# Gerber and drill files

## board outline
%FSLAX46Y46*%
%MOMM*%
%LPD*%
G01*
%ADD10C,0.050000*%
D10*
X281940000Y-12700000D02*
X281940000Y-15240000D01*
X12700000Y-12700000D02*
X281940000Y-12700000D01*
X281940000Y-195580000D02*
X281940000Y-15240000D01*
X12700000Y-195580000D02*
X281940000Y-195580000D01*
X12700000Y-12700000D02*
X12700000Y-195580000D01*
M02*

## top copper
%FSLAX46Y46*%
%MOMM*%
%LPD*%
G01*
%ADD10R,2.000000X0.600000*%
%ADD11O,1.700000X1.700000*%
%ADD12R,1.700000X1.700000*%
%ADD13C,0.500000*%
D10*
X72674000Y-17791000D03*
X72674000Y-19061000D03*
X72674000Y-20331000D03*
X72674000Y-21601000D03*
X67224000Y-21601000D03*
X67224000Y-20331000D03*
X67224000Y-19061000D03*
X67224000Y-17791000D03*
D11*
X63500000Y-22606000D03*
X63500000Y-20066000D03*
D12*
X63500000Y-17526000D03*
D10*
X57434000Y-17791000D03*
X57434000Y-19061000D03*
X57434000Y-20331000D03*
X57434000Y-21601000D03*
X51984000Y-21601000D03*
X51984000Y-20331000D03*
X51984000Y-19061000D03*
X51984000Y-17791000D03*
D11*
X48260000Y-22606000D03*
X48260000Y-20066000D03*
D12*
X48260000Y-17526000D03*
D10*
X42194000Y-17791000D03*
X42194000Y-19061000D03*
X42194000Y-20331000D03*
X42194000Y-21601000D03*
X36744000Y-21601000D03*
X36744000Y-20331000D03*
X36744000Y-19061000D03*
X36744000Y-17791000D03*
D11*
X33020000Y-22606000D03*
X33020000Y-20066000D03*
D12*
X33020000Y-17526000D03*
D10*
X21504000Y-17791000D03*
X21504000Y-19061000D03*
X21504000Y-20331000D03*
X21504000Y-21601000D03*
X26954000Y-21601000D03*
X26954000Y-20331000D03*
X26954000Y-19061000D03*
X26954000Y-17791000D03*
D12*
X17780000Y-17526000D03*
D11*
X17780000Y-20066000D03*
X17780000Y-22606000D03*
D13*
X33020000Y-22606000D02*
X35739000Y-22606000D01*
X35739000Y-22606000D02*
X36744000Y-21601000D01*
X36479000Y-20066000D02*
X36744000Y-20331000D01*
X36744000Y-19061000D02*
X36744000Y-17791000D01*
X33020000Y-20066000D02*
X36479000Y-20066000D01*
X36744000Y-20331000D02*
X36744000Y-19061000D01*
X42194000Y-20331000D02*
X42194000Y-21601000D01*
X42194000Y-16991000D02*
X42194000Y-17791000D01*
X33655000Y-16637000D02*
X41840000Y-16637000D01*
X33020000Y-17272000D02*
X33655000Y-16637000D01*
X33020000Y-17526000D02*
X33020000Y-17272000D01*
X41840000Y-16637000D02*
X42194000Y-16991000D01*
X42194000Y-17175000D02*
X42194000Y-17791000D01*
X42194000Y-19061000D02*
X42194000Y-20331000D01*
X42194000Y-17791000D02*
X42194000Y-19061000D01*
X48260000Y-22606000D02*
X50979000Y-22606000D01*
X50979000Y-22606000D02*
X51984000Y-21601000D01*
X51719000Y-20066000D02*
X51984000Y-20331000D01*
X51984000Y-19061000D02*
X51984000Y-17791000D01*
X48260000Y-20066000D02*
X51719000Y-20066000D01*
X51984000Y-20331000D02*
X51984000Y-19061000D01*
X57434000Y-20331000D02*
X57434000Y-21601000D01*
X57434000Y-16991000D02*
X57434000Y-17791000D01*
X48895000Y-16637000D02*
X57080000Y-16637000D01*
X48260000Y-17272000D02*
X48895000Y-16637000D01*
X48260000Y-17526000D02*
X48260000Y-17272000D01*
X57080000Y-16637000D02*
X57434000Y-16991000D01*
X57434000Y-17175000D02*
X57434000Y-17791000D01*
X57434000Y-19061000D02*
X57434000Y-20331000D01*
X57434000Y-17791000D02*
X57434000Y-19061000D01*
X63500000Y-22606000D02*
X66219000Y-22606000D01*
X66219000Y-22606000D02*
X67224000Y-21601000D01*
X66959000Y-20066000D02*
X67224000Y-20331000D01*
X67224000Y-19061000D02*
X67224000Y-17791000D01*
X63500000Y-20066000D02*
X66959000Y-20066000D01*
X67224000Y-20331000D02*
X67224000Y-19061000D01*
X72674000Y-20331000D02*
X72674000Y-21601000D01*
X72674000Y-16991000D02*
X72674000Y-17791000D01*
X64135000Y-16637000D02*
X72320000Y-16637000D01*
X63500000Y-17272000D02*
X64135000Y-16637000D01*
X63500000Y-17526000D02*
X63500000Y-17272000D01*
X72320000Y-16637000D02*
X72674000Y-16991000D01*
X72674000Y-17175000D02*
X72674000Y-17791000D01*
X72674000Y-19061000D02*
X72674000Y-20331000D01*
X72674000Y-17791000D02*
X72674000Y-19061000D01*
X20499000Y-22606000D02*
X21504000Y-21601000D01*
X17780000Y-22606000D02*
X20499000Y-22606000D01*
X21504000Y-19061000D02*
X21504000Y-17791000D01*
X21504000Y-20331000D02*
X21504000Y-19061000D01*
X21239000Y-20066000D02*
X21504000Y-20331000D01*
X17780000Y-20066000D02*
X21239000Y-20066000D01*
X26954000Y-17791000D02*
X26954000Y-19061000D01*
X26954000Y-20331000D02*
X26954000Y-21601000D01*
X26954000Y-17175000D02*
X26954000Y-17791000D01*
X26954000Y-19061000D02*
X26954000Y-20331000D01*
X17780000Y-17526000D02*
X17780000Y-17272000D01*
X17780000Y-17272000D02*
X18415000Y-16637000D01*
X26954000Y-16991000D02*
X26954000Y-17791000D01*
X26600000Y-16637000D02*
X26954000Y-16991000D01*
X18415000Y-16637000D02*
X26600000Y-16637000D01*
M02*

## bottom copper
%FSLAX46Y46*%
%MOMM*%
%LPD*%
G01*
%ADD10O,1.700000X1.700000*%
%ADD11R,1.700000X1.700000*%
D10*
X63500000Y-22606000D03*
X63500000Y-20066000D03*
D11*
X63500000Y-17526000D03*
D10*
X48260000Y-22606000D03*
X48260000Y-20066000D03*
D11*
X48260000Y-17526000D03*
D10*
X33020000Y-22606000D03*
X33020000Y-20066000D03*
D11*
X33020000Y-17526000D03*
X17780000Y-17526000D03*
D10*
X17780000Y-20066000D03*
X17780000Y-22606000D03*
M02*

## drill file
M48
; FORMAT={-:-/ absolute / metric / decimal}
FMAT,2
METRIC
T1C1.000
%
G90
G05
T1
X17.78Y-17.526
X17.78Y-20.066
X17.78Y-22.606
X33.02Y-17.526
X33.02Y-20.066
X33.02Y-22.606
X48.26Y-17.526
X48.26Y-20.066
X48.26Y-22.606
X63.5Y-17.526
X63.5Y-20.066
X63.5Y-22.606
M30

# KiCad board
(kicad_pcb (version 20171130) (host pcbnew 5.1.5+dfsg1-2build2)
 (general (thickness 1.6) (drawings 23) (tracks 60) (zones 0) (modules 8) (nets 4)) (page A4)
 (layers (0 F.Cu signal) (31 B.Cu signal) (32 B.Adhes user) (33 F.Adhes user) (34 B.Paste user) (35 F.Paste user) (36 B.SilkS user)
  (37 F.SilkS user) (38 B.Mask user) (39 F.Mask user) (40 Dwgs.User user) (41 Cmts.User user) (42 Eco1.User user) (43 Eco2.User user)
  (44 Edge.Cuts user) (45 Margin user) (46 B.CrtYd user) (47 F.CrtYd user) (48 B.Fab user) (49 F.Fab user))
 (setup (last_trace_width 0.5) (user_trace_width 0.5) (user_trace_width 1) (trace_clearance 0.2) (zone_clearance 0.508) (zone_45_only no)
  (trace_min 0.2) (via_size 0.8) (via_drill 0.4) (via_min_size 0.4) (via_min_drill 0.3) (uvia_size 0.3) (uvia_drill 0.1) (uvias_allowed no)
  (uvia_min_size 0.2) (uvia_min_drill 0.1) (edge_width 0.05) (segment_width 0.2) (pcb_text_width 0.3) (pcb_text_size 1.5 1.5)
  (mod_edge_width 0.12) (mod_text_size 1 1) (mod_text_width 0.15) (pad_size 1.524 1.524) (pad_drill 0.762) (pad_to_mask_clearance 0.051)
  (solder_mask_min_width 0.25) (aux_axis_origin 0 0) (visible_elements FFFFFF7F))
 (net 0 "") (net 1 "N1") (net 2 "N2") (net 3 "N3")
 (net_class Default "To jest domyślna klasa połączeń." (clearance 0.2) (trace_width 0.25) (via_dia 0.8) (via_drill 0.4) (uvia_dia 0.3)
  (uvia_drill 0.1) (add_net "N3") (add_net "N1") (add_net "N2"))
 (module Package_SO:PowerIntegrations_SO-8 (layer F.Cu) (at 69.949 19.696)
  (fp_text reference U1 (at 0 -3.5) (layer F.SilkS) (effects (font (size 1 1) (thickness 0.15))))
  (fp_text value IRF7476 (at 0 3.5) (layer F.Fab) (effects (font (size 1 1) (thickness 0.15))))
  (pad 8 smd rect (at 2.725 -1.905) (size 2 0.6) (layers F.Cu F.Paste F.Mask))
  (pad 7 smd rect (at 2.725 -0.635) (size 2 0.6) (layers F.Cu F.Paste F.Mask))
  (pad 6 smd rect (at 2.725 0.635) (size 2 0.6) (layers F.Cu F.Paste F.Mask))
  (pad 5 smd rect (at 2.725 1.905) (size 2 0.6) (layers F.Cu F.Paste F.Mask))
  (pad 4 smd rect (at -2.725 1.905) (size 2 0.6) (layers F.Cu F.Paste F.Mask))
  (pad 3 smd rect (at -2.725 0.635) (size 2 0.6) (layers F.Cu F.Paste F.Mask))
  (pad 2 smd rect (at -2.725 -0.635) (size 2 0.6) (layers F.Cu F.Paste F.Mask))
  (pad 1 smd rect (at -2.725 -1.905) (size 2 0.6) (layers F.Cu F.Paste F.Mask)))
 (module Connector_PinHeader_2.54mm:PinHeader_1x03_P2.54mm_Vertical (layer B.Cu) (at 63.5 17.526 180)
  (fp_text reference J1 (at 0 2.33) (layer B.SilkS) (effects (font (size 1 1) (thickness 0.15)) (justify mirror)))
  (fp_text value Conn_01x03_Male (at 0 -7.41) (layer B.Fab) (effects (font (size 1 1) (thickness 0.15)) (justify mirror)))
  (pad 3 thru_hole oval (at 0 -5.08 180) (size 1.7 1.7) (drill 1) (layers *.Cu *.Mask))
  (pad 2 thru_hole oval (at 0 -2.54 180) (size 1.7 1.7) (drill 1) (layers *.Cu *.Mask))
  (pad 1 thru_hole rect (at 0 0 180) (size 1.7 1.7) (drill 1) (layers *.Cu *.Mask)))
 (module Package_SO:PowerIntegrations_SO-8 (layer F.Cu) (at 54.709 19.696)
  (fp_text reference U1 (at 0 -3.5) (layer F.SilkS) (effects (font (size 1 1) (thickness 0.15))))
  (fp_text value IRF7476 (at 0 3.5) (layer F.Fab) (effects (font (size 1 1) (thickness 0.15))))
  (pad 8 smd rect (at 2.725 -1.905) (size 2 0.6) (layers F.Cu F.Paste F.Mask))
  (pad 7 smd rect (at 2.725 -0.635) (size 2 0.6) (layers F.Cu F.Paste F.Mask))
  (pad 6 smd rect (at 2.725 0.635) (size 2 0.6) (layers F.Cu F.Paste F.Mask))
  (pad 5 smd rect (at 2.725 1.905) (size 2 0.6) (layers F.Cu F.Paste F.Mask))
  (pad 4 smd rect (at -2.725 1.905) (size 2 0.6) (layers F.Cu F.Paste F.Mask))
  (pad 3 smd rect (at -2.725 0.635) (size 2 0.6) (layers F.Cu F.Paste F.Mask))
  (pad 2 smd rect (at -2.725 -0.635) (size 2 0.6) (layers F.Cu F.Paste F.Mask))
  (pad 1 smd rect (at -2.725 -1.905) (size 2 0.6) (layers F.Cu F.Paste F.Mask)))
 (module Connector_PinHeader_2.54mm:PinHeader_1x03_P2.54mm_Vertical (layer B.Cu) (at 48.26 17.526 180)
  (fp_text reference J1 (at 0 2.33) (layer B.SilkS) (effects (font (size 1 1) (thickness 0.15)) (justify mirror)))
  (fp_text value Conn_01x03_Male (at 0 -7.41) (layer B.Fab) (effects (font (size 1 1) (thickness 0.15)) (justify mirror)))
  (pad 3 thru_hole oval (at 0 -5.08 180) (size 1.7 1.7) (drill 1) (layers *.Cu *.Mask))
  (pad 2 thru_hole oval (at 0 -2.54 180) (size 1.7 1.7) (drill 1) (layers *.Cu *.Mask))
  (pad 1 thru_hole rect (at 0 0 180) (size 1.7 1.7) (drill 1) (layers *.Cu *.Mask)))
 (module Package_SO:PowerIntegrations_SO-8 (layer F.Cu) (at 39.469 19.696)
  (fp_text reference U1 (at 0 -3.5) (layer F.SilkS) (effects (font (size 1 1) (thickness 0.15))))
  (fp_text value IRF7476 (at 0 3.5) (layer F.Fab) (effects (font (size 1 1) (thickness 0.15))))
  (pad 8 smd rect (at 2.725 -1.905) (size 2 0.6) (layers F.Cu F.Paste F.Mask))
  (pad 7 smd rect (at 2.725 -0.635) (size 2 0.6) (layers F.Cu F.Paste F.Mask))
  (pad 6 smd rect (at 2.725 0.635) (size 2 0.6) (layers F.Cu F.Paste F.Mask))
  (pad 5 smd rect (at 2.725 1.905) (size 2 0.6) (layers F.Cu F.Paste F.Mask))
  (pad 4 smd rect (at -2.725 1.905) (size 2 0.6) (layers F.Cu F.Paste F.Mask))
  (pad 3 smd rect (at -2.725 0.635) (size 2 0.6) (layers F.Cu F.Paste F.Mask))
  (pad 2 smd rect (at -2.725 -0.635) (size 2 0.6) (layers F.Cu F.Paste F.Mask))
  (pad 1 smd rect (at -2.725 -1.905) (size 2 0.6) (layers F.Cu F.Paste F.Mask)))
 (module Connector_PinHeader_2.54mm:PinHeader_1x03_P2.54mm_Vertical (layer B.Cu) (at 33.02 17.526 180)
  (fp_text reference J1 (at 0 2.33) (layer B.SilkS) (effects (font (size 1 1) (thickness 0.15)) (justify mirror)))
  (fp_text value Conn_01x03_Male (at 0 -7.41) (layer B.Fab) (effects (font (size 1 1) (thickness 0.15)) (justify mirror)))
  (pad 3 thru_hole oval (at 0 -5.08 180) (size 1.7 1.7) (drill 1) (layers *.Cu *.Mask))
  (pad 2 thru_hole oval (at 0 -2.54 180) (size 1.7 1.7) (drill 1) (layers *.Cu *.Mask))
  (pad 1 thru_hole rect (at 0 0 180) (size 1.7 1.7) (drill 1) (layers *.Cu *.Mask)))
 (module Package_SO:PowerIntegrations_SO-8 (layer F.Cu) (at 24.229 19.696)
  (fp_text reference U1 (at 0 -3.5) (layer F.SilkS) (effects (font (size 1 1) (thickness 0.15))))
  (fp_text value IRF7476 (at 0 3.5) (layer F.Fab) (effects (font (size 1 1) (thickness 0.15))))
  (pad 1 smd rect (at -2.725 -1.905) (size 2 0.6) (layers F.Cu F.Paste F.Mask) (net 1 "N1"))
  (pad 2 smd rect (at -2.725 -0.635) (size 2 0.6) (layers F.Cu F.Paste F.Mask) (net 1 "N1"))
  (pad 3 smd rect (at -2.725 0.635) (size 2 0.6) (layers F.Cu F.Paste F.Mask) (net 1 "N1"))
  (pad 4 smd rect (at -2.725 1.905) (size 2 0.6) (layers F.Cu F.Paste F.Mask) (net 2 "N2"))
  (pad 5 smd rect (at 2.725 1.905) (size 2 0.6) (layers F.Cu F.Paste F.Mask) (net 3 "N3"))
  (pad 6 smd rect (at 2.725 0.635) (size 2 0.6) (layers F.Cu F.Paste F.Mask) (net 3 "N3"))
  (pad 7 smd rect (at 2.725 -0.635) (size 2 0.6) (layers F.Cu F.Paste F.Mask) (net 3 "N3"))
  (pad 8 smd rect (at 2.725 -1.905) (size 2 0.6) (layers F.Cu F.Paste F.Mask) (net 3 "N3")))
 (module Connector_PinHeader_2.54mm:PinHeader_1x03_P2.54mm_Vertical (layer B.Cu) (at 17.78 17.526 180)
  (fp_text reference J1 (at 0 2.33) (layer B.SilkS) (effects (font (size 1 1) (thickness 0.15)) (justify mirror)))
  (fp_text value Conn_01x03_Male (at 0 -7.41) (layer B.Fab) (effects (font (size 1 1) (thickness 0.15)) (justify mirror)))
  (pad 1 thru_hole rect (at 0 0 180) (size 1.7 1.7) (drill 1) (layers *.Cu *.Mask) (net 3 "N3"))
  (pad 2 thru_hole oval (at 0 -2.54 180) (size 1.7 1.7) (drill 1) (layers *.Cu *.Mask) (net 1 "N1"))
  (pad 3 thru_hole oval (at 0 -5.08 180) (size 1.7 1.7) (drill 1) (layers *.Cu *.Mask) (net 2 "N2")))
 (gr_line (start 281.94 12.7) (end 281.94 15.24) (layer Edge.Cuts) (width 0.05))
 (gr_line (start 12.7 12.7) (end 281.94 12.7) (layer Edge.Cuts) (width 0.05))
 (gr_line (start 281.94 195.58) (end 281.94 15.24) (layer Edge.Cuts) (width 0.05))
 (gr_line (start 12.7 195.58) (end 281.94 195.58) (layer Edge.Cuts) (width 0.05))
 (gr_line (start 12.7 12.7) (end 12.7 195.58) (layer Edge.Cuts) (width 0.05))
 (segment (start 33.02 22.606) (end 35.739 22.606) (width 0.5) (layer F.Cu) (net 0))
 (segment (start 35.739 22.606) (end 36.744 21.601) (width 0.5) (layer F.Cu) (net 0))
 (segment (start 36.479 20.066) (end 36.744 20.331) (width 0.5) (layer F.Cu) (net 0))
 (segment (start 36.744 19.061) (end 36.744 17.791) (width 0.5) (layer F.Cu) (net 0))
 (segment (start 33.02 20.066) (end 36.479 20.066) (width 0.5) (layer F.Cu) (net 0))
 (segment (start 36.744 20.331) (end 36.744 19.061) (width 0.5) (layer F.Cu) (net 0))
 (segment (start 42.194 20.331) (end 42.194 21.601) (width 0.5) (layer F.Cu) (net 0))
 (segment (start 42.194 16.991) (end 42.194 17.791) (width 0.5) (layer F.Cu) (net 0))
 (segment (start 33.655 16.637) (end 41.84 16.637) (width 0.5) (layer F.Cu) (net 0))
 (segment (start 33.02 17.272) (end 33.655 16.637) (width 0.5) (layer F.Cu) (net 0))
 (segment (start 33.02 17.526) (end 33.02 17.272) (width 0.5) (layer F.Cu) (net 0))
 (segment (start 41.84 16.637) (end 42.194 16.991) (width 0.5) (layer F.Cu) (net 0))
 (segment (start 42.194 17.175) (end 42.194 17.791) (width 0.5) (layer F.Cu) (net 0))
 (segment (start 42.194 19.061) (end 42.194 20.331) (width 0.5) (layer F.Cu) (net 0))
 (segment (start 42.194 17.791) (end 42.194 19.061) (width 0.5) (layer F.Cu) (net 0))
 (segment (start 48.26 22.606) (end 50.979 22.606) (width 0.5) (layer F.Cu) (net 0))
 (segment (start 50.979 22.606) (end 51.984 21.601) (width 0.5) (layer F.Cu) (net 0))
 (segment (start 51.719 20.066) (end 51.984 20.331) (width 0.5) (layer F.Cu) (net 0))
 (segment (start 51.984 19.061) (end 51.984 17.791) (width 0.5) (layer F.Cu) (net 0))
 (segment (start 48.26 20.066) (end 51.719 20.066) (width 0.5) (layer F.Cu) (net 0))
 (segment (start 51.984 20.331) (end 51.984 19.061) (width 0.5) (layer F.Cu) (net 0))
 (segment (start 57.434 20.331) (end 57.434 21.601) (width 0.5) (layer F.Cu) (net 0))
 (segment (start 57.434 16.991) (end 57.434 17.791) (width 0.5) (layer F.Cu) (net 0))
 (segment (start 48.895 16.637) (end 57.08 16.637) (width 0.5) (layer F.Cu) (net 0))
 (segment (start 48.26 17.272) (end 48.895 16.637) (width 0.5) (layer F.Cu) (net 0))
 (segment (start 48.26 17.526) (end 48.26 17.272) (width 0.5) (layer F.Cu) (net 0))
 (segment (start 57.08 16.637) (end 57.434 16.991) (width 0.5) (layer F.Cu) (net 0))
 (segment (start 57.434 17.175) (end 57.434 17.791) (width 0.5) (layer F.Cu) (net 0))
 (segment (start 57.434 19.061) (end 57.434 20.331) (width 0.5) (layer F.Cu) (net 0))
 (segment (start 57.434 17.791) (end 57.434 19.061) (width 0.5) (layer F.Cu) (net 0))
 (segment (start 63.5 22.606) (end 66.219 22.606) (width 0.5) (layer F.Cu) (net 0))
 (segment (start 66.219 22.606) (end 67.224 21.601) (width 0.5) (layer F.Cu) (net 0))
 (segment (start 66.959 20.066) (end 67.224 20.331) (width 0.5) (layer F.Cu) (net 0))
 (segment (start 67.224 19.061) (end 67.224 17.791) (width 0.5) (layer F.Cu) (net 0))
 (segment (start 63.5 20.066) (end 66.959 20.066) (width 0.5) (layer F.Cu) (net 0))
 (segment (start 67.224 20.331) (end 67.224 19.061) (width 0.5) (layer F.Cu) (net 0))
 (segment (start 72.674 20.331) (end 72.674 21.601) (width 0.5) (layer F.Cu) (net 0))
 (segment (start 72.674 16.991) (end 72.674 17.791) (width 0.5) (layer F.Cu) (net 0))
 (segment (start 64.135 16.637) (end 72.32 16.637) (width 0.5) (layer F.Cu) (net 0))
 (segment (start 63.5 17.272) (end 64.135 16.637) (width 0.5) (layer F.Cu) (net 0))
 (segment (start 63.5 17.526) (end 63.5 17.272) (width 0.5) (layer F.Cu) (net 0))
 (segment (start 72.32 16.637) (end 72.674 16.991) (width 0.5) (layer F.Cu) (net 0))
 (segment (start 72.674 17.175) (end 72.674 17.791) (width 0.5) (layer F.Cu) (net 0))
 (segment (start 72.674 19.061) (end 72.674 20.331) (width 0.5) (layer F.Cu) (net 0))
 (segment (start 72.674 17.791) (end 72.674 19.061) (width 0.5) (layer F.Cu) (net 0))
 (segment (start 20.499 22.606) (end 21.504 21.601) (width 0.5) (layer F.Cu) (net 2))
 (segment (start 17.78 22.606) (end 20.499 22.606) (width 0.5) (layer F.Cu) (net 2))
 (segment (start 21.504 19.061) (end 21.504 17.791) (width 0.5) (layer F.Cu) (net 1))
 (segment (start 21.504 20.331) (end 21.504 19.061) (width 0.5) (layer F.Cu) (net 1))
 (segment (start 21.239 20.066) (end 21.504 20.331) (width 0.5) (layer F.Cu) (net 1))
 (segment (start 17.78 20.066) (end 21.239 20.066) (width 0.5) (layer F.Cu) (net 1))
 (segment (start 26.954 17.791) (end 26.954 19.061) (width 0.5) (layer F.Cu) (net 3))
 (segment (start 26.954 20.331) (end 26.954 21.601) (width 0.5) (layer F.Cu) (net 3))
 (segment (start 26.954 17.175) (end 26.954 17.791) (width 0.5) (layer F.Cu) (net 3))
 (segment (start 26.954 19.061) (end 26.954 20.331) (width 0.5) (layer F.Cu) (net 3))
 (segment (start 17.78 17.526) (end 17.78 17.272) (width 0.5) (layer F.Cu) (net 3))
 (segment (start 17.78 17.272) (end 18.415 16.637) (width 0.5) (layer F.Cu) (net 3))
 (segment (start 26.954 16.991) (end 26.954 17.791) (width 0.5) (layer F.Cu) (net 3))
 (segment (start 26.6 16.637) (end 26.954 16.991) (width 0.5) (layer F.Cu) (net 3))
 (segment (start 18.415 16.637) (end 26.6 16.637) (width 0.5) (layer F.Cu) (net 3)))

